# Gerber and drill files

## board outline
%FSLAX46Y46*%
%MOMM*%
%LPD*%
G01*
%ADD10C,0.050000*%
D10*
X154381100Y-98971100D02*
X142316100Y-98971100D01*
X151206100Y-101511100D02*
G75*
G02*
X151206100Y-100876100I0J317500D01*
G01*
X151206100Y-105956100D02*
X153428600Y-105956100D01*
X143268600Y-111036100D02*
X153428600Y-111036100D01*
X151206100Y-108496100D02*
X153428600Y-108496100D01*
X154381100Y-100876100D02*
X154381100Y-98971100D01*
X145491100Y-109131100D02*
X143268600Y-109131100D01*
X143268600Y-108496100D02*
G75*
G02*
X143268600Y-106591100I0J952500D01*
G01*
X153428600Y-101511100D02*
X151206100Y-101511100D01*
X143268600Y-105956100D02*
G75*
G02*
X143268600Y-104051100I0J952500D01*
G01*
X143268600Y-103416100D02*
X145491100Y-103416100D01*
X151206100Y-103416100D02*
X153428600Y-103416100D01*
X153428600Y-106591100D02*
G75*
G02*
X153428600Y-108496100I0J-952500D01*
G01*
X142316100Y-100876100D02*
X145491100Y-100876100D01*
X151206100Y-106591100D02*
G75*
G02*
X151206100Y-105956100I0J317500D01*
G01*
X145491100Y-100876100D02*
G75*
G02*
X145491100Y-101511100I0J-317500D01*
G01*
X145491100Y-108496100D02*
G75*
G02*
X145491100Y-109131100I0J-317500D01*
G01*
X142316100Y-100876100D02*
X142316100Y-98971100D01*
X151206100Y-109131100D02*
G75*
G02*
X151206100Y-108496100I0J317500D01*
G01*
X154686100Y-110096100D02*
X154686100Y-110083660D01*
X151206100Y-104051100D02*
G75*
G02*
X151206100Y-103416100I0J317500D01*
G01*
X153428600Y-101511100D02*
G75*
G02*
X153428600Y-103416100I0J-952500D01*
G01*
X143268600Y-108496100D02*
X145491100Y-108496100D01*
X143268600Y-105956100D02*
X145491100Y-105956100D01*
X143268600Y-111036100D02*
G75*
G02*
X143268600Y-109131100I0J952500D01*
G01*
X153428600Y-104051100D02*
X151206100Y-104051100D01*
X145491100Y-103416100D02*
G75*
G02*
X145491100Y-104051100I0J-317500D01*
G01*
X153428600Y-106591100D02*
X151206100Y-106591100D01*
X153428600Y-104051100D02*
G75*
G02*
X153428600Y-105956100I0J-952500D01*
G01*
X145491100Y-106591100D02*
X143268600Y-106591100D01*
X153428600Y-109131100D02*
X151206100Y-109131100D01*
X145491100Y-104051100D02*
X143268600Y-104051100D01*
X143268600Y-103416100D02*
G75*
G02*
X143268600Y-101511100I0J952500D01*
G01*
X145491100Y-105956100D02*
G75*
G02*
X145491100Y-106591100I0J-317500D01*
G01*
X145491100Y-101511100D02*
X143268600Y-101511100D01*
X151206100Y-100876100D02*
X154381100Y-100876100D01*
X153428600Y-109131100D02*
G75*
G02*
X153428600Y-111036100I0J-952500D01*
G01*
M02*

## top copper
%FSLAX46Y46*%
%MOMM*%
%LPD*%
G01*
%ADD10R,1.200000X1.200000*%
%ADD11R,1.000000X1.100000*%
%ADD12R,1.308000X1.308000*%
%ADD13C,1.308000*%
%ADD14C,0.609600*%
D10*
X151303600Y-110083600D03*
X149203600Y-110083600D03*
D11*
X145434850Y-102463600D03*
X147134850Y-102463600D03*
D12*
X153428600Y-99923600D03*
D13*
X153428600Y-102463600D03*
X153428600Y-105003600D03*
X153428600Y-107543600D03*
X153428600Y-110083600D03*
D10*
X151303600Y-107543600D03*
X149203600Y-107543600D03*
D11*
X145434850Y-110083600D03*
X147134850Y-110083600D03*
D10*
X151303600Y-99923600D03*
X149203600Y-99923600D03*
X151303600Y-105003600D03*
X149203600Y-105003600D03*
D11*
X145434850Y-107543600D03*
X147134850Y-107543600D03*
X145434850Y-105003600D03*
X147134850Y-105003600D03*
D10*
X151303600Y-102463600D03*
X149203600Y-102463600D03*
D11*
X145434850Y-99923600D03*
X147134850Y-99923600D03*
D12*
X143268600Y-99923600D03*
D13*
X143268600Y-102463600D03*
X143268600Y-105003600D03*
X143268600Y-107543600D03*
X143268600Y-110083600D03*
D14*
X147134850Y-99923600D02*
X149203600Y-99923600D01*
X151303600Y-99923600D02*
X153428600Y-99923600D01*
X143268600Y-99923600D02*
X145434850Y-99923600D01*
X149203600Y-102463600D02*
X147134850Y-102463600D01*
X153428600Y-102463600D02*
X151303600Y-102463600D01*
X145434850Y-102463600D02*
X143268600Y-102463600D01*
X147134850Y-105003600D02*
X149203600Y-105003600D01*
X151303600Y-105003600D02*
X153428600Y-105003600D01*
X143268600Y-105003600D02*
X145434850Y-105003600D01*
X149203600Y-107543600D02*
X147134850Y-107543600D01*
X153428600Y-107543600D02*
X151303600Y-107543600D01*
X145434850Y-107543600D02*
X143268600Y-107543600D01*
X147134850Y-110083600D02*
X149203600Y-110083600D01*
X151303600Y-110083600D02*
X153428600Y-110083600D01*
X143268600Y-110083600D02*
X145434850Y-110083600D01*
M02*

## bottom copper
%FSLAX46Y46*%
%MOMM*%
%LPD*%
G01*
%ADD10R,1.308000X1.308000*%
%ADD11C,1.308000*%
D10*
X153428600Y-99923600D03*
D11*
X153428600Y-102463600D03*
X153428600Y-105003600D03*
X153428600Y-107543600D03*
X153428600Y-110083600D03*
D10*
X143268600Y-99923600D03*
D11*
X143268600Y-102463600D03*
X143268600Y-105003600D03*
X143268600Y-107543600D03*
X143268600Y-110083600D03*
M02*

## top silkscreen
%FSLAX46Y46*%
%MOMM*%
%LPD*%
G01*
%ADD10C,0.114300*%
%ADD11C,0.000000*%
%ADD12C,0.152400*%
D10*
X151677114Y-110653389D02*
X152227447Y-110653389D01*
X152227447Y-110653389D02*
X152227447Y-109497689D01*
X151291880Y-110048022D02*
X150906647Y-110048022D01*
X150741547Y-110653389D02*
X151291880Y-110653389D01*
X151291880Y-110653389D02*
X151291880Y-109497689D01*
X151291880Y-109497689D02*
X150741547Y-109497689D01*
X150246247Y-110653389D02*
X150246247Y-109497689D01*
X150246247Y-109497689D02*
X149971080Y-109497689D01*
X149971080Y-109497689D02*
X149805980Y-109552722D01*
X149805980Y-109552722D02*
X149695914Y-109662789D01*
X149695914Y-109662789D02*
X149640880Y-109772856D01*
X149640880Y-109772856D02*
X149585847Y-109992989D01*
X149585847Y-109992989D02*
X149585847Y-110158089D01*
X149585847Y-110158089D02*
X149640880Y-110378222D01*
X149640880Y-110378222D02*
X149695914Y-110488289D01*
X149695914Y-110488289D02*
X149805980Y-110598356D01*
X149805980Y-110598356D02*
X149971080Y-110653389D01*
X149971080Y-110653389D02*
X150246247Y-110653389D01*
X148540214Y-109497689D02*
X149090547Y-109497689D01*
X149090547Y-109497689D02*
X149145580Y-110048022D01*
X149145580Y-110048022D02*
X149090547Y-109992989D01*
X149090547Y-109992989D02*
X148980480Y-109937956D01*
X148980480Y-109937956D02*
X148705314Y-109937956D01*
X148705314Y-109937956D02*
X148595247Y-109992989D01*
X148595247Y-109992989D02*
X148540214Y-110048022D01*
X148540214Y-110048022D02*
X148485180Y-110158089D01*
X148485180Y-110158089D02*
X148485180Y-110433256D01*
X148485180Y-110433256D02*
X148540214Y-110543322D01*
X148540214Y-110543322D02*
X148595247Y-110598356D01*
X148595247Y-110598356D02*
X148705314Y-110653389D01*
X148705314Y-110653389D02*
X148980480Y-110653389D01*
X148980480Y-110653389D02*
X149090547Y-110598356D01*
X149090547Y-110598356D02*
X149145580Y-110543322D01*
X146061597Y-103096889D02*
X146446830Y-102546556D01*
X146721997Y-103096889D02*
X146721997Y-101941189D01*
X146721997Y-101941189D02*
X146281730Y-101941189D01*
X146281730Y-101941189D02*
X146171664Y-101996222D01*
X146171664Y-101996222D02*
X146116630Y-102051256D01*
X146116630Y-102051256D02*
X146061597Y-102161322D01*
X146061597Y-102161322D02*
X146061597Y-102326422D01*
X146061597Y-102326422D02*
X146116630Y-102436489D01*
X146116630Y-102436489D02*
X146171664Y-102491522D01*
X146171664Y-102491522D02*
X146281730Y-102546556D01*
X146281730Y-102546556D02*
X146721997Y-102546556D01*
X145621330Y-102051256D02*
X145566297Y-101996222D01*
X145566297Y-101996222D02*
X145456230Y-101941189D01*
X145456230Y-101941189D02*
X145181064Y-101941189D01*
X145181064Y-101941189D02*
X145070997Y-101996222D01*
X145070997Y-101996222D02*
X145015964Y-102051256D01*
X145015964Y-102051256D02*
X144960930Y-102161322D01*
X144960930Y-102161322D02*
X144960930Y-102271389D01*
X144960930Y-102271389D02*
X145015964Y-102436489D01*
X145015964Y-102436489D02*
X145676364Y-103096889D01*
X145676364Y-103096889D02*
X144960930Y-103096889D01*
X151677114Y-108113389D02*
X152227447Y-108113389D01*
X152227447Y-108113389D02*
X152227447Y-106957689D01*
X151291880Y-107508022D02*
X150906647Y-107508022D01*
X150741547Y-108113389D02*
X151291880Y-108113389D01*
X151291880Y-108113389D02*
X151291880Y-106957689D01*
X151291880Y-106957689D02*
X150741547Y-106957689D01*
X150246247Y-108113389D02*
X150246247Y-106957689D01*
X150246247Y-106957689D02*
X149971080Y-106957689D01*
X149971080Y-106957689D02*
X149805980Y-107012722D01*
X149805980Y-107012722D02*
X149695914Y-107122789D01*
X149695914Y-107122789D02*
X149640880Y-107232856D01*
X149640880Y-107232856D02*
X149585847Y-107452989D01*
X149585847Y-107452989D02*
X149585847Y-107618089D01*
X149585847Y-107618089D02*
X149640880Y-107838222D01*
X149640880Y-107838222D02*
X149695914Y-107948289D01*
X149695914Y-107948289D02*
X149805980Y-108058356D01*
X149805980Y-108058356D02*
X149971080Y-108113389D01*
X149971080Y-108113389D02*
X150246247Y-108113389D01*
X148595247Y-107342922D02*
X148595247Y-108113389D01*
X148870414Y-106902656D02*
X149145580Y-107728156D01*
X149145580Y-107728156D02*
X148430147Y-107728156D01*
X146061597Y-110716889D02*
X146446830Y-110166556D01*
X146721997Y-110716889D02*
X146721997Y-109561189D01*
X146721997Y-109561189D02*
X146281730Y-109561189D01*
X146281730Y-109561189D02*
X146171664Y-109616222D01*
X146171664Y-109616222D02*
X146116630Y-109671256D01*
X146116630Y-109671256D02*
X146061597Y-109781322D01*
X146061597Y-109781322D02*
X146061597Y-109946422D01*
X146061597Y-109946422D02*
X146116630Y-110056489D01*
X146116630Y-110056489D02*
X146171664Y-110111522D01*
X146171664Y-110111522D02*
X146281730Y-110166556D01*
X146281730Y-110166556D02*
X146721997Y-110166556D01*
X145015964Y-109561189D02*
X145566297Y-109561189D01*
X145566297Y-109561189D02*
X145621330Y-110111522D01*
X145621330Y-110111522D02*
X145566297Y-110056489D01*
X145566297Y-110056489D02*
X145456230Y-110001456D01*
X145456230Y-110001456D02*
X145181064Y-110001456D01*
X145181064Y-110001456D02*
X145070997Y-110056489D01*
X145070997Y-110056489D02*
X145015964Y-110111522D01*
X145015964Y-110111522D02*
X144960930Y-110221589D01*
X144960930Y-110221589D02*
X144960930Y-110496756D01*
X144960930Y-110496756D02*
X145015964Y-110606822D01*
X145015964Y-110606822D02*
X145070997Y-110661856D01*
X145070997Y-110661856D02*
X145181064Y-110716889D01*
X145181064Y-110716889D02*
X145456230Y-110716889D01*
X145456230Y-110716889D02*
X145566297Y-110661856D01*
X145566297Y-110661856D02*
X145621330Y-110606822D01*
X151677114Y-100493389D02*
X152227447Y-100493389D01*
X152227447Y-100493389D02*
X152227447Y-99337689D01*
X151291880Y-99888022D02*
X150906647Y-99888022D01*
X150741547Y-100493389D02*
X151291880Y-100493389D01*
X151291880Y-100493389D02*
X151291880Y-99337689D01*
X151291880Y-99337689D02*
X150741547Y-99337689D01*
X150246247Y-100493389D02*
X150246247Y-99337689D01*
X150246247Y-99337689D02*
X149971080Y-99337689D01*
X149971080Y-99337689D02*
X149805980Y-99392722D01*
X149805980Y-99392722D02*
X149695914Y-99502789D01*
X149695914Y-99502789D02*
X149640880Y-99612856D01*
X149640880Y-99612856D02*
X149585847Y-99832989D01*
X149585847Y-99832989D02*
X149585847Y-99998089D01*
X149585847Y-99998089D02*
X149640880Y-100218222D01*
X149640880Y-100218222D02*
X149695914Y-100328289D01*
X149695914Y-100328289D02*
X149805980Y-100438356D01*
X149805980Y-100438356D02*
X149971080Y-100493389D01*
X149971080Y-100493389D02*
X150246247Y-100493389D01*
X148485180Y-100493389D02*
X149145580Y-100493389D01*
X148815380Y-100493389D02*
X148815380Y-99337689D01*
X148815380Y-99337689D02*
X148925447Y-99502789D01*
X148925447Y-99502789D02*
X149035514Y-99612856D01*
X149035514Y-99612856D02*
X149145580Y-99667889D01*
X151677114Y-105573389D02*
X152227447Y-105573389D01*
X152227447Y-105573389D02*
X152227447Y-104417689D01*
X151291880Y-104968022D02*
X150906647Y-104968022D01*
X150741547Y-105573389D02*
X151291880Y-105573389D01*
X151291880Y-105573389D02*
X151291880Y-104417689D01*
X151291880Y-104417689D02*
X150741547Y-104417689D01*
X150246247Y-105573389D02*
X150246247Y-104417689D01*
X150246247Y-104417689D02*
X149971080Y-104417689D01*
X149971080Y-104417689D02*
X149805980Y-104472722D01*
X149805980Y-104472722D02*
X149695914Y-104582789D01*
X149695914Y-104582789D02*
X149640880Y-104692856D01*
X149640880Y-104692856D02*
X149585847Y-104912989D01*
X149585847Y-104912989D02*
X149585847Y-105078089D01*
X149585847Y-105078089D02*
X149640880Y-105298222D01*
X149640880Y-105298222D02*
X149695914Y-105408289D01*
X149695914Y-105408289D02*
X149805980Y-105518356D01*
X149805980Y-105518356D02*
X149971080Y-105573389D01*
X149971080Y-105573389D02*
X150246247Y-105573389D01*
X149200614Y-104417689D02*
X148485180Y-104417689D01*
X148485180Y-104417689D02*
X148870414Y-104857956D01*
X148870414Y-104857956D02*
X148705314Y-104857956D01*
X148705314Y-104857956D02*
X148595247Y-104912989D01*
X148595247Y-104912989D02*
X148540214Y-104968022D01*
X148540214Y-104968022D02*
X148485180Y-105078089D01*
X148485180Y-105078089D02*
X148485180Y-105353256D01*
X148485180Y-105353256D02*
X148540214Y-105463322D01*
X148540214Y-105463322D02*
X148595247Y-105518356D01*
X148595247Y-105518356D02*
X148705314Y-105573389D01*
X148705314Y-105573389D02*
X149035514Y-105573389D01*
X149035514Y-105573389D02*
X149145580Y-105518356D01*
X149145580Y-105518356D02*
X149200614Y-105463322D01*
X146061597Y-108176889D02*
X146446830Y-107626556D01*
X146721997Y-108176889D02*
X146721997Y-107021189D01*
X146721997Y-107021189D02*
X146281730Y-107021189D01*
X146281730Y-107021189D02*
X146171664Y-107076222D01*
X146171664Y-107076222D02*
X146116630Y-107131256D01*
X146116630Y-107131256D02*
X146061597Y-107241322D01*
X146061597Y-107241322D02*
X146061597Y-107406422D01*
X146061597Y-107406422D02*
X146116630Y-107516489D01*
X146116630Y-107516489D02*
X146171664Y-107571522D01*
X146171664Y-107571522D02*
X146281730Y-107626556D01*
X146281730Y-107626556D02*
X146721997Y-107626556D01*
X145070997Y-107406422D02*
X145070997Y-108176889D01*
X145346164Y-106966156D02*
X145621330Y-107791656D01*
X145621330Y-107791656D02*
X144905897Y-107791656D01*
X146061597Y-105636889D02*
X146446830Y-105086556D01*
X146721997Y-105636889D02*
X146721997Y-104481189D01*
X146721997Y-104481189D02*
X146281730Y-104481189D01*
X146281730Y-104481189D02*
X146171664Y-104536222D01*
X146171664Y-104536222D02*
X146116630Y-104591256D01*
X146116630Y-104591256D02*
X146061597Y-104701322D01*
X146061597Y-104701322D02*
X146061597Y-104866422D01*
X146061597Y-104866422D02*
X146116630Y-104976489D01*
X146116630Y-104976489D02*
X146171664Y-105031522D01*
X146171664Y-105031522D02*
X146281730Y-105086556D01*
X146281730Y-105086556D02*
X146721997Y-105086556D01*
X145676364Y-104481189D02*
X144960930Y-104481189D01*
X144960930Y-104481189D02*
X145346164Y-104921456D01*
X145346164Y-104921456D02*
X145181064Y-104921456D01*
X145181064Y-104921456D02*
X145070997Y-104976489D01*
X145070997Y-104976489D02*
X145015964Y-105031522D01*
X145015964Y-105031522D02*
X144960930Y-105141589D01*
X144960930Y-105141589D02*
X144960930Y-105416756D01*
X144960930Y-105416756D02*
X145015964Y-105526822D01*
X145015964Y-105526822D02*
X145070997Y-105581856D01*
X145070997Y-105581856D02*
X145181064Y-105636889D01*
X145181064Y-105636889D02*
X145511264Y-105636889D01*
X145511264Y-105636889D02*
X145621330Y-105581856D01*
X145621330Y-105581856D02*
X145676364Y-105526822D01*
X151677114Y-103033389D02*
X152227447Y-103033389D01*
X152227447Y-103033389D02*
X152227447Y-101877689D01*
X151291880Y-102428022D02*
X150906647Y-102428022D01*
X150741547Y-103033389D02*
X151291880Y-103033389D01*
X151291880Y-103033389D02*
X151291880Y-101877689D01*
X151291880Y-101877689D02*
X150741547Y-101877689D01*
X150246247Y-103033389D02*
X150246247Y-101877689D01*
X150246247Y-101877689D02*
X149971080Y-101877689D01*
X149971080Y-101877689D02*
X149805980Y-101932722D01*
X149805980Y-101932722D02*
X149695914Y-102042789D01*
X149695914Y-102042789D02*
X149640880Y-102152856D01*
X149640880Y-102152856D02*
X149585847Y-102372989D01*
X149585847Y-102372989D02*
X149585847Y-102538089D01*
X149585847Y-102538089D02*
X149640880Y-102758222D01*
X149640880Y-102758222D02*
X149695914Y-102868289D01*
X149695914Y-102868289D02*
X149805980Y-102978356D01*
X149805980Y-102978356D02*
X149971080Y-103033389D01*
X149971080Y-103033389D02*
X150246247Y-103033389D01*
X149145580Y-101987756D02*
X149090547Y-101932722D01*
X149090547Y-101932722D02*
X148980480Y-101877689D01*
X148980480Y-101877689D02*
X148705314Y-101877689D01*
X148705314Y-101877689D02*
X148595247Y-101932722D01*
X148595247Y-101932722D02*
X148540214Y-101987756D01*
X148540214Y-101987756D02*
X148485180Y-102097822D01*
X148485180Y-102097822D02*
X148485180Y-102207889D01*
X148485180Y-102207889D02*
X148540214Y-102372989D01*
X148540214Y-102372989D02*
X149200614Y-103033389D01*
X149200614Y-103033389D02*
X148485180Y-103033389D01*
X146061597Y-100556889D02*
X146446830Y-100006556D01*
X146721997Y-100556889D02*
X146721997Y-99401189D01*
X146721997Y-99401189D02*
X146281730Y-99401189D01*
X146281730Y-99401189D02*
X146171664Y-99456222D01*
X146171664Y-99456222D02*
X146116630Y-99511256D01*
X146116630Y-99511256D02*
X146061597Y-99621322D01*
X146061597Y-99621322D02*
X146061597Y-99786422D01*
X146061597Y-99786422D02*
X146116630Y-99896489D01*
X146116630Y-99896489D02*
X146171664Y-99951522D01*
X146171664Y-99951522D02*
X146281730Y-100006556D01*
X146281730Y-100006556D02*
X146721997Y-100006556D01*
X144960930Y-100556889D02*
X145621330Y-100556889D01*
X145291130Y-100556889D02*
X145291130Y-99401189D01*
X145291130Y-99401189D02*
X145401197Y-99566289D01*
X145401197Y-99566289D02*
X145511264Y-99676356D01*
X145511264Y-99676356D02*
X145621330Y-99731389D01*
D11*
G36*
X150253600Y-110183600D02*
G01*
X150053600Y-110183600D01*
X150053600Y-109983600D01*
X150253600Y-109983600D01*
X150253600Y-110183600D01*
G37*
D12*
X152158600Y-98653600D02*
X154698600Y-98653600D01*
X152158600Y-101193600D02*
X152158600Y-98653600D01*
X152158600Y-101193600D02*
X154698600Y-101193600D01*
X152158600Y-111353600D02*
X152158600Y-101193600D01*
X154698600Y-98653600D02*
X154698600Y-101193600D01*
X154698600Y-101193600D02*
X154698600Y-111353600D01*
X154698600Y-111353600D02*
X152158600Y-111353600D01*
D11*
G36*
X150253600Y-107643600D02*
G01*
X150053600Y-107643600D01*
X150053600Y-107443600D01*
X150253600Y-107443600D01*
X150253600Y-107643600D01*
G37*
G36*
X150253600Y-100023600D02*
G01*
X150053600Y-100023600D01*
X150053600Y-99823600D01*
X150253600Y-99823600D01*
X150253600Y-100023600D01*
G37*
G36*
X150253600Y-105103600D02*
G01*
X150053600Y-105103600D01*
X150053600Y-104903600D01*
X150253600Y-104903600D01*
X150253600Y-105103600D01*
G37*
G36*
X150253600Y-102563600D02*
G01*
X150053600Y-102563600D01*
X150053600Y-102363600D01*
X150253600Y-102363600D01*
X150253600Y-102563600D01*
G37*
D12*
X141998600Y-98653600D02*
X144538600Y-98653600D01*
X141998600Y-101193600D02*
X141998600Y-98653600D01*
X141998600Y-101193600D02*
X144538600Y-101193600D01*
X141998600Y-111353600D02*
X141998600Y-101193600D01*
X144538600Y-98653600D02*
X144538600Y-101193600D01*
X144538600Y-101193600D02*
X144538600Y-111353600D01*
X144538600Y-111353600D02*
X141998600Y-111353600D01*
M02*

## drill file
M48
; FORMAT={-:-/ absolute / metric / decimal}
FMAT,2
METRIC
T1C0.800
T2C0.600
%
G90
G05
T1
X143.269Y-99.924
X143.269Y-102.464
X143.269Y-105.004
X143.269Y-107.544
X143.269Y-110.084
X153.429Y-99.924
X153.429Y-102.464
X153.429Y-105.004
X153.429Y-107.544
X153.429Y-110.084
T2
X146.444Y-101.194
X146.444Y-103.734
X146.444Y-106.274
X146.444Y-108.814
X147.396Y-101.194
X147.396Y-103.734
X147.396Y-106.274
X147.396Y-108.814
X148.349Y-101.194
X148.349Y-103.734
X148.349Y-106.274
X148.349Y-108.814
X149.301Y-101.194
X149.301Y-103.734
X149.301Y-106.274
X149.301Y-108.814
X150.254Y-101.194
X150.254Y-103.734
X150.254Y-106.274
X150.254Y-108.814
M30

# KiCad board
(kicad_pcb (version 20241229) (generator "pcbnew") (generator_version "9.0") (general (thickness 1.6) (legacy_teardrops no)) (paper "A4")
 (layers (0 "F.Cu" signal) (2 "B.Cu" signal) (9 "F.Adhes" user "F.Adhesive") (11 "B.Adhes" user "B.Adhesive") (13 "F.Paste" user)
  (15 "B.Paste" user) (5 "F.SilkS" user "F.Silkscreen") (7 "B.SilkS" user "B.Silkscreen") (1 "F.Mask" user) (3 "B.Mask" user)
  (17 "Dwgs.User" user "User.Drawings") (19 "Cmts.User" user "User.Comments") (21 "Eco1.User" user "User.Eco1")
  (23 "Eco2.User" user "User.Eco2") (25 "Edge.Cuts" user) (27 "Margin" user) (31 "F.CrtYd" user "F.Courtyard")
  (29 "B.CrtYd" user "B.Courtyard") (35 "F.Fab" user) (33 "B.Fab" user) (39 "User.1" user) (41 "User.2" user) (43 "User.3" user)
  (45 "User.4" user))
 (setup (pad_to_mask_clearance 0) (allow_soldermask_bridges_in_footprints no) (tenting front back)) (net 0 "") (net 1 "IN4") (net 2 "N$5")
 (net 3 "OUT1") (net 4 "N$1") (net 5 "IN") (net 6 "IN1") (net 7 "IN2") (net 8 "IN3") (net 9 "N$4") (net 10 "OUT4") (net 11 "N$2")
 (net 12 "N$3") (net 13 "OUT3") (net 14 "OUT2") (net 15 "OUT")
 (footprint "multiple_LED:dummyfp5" (layer "F.Cu") (at 148.3486 103.7336)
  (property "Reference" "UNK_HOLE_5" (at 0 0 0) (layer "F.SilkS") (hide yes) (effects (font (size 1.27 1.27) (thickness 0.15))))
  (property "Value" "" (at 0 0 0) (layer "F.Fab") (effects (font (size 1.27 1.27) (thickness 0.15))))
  (pad "" np_thru_hole circle (at 0 0) (size 0.6 0.6) (drill 0.6) (layers "*.Cu" "*.Mask")))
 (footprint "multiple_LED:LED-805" (layer "F.Cu") (at 150.2536 110.0836 90)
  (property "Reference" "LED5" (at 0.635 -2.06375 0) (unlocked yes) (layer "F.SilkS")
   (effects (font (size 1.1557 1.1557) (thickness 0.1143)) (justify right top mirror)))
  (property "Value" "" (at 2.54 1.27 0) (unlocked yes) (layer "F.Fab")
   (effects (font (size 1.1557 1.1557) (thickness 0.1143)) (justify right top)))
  (fp_poly (pts (xy -0.1 0) (xy 0.1 0) (xy 0.1 -0.2) (xy -0.1 -0.2)) (stroke (width 0) (type default)) (fill yes) (layer "F.SilkS"))
  (pad "A" smd rect (at 0 1.05 90) (size 1.2 1.2) (layers "F.Cu" "F.Mask" "F.Paste") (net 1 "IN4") (solder_mask_margin 0.0508)
   (solder_paste_margin 0) (thermal_bridge_angle 0))
  (pad "C" smd rect (at 0 -1.05 90) (size 1.2 1.2) (layers "F.Cu" "F.Mask" "F.Paste") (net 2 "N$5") (solder_mask_margin 0.0508)
   (solder_paste_margin 0) (thermal_bridge_angle 0)))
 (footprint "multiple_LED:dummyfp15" (layer "F.Cu") (at 148.3486 108.8136)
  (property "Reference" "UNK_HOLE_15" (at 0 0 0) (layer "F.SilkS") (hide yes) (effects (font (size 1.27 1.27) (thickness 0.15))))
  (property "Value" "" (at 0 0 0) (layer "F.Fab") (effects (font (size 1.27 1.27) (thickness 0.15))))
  (pad "" np_thru_hole circle (at 0 0) (size 0.6 0.6) (drill 0.6) (layers "*.Cu" "*.Mask")))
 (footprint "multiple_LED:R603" (layer "F.Cu") (at 146.28485 102.4636)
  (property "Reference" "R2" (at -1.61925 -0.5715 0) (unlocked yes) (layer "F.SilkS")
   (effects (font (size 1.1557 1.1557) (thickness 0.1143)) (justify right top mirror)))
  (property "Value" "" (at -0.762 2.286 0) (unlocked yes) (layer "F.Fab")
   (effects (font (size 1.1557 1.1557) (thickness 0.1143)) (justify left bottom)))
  (pad "1" smd rect (at -0.85 0) (size 1 1.1) (layers "F.Cu" "F.Mask" "F.Paste") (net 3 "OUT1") (solder_mask_margin 0.0508)
   (solder_paste_margin 0) (thermal_bridge_angle 0))
  (pad "2" smd rect (at 0.85 0) (size 1 1.1) (layers "F.Cu" "F.Mask" "F.Paste") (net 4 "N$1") (solder_mask_margin 0.0508)
   (solder_paste_margin 0) (thermal_bridge_angle 0)))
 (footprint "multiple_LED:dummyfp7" (layer "F.Cu") (at 149.3011 103.7336)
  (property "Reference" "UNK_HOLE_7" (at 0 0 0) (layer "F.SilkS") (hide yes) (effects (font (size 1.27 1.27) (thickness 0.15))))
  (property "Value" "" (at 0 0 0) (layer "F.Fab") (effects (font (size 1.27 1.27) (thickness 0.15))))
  (pad "" np_thru_hole circle (at 0 0) (size 0.6 0.6) (drill 0.6) (layers "*.Cu" "*.Mask")))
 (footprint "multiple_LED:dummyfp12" (layer "F.Cu") (at 149.3011 106.2736)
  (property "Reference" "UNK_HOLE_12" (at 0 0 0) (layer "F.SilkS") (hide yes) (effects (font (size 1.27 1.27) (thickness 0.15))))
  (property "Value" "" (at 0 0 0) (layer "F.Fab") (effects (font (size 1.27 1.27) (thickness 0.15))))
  (pad "" np_thru_hole circle (at 0 0) (size 0.6 0.6) (drill 0.6) (layers "*.Cu" "*.Mask")))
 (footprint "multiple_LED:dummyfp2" (layer "F.Cu") (at 149.3011 101.1936)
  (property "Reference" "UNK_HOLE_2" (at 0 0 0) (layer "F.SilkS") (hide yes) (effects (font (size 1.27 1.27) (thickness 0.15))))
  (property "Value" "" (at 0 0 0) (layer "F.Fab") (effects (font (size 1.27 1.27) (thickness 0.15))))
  (pad "" np_thru_hole circle (at 0 0) (size 0.6 0.6) (drill 0.6) (layers "*.Cu" "*.Mask")))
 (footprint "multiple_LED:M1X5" (layer "F.Cu") (at 153.4286 105.0036 -90)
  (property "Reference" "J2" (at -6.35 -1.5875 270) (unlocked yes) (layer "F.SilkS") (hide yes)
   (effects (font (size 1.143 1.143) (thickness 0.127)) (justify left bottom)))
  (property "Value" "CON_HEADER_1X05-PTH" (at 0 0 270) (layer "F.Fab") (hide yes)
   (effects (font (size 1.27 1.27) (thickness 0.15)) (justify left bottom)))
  (fp_line (start -6.35 1.27) (end -6.35 -1.27) (stroke (width 0.1524) (type solid)) (layer "F.SilkS"))
  (fp_line (start -3.81 1.27) (end -6.35 1.27) (stroke (width 0.1524) (type solid)) (layer "F.SilkS"))
  (fp_line (start -3.81 1.27) (end -3.81 -1.27) (stroke (width 0.1524) (type solid)) (layer "F.SilkS"))
  (fp_line (start 6.35 1.27) (end -3.81 1.27) (stroke (width 0.1524) (type solid)) (layer "F.SilkS"))
  (fp_line (start -6.35 -1.27) (end -3.81 -1.27) (stroke (width 0.1524) (type solid)) (layer "F.SilkS"))
  (fp_line (start -3.81 -1.27) (end 6.35 -1.27) (stroke (width 0.1524) (type solid)) (layer "F.SilkS"))
  (fp_line (start 6.35 -1.27) (end 6.35 1.27) (stroke (width 0.1524) (type solid)) (layer "F.SilkS"))
  (pad "1" thru_hole rect (at -5.08 0 270) (size 1.308 1.308) (drill 0.8) (layers "*.Cu" "*.Mask") (remove_unused_layers no) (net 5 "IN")
   (solder_mask_margin 0.0508) (thermal_bridge_angle 0))
  (pad "2" thru_hole circle (at -2.54 0 270) (size 1.308 1.308) (drill 0.8) (layers "*.Cu" "*.Mask") (remove_unused_layers no) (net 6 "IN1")
   (solder_mask_margin 0.0508) (thermal_bridge_angle 0))
  (pad "3" thru_hole circle (at 0 0 270) (size 1.308 1.308) (drill 0.8) (layers "*.Cu" "*.Mask") (remove_unused_layers no) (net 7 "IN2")
   (solder_mask_margin 0.0508) (thermal_bridge_angle 0))
  (pad "4" thru_hole circle (at 2.54 0 270) (size 1.308 1.308) (drill 0.8) (layers "*.Cu" "*.Mask") (remove_unused_layers no) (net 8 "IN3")
   (solder_mask_margin 0.0508) (thermal_bridge_angle 0))
  (pad "5" thru_hole circle (at 5.08 0 270) (size 1.308 1.308) (drill 0.8) (layers "*.Cu" "*.Mask") (remove_unused_layers no) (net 1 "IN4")
   (solder_mask_margin 0.0508) (thermal_bridge_angle 0)))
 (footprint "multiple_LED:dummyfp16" (layer "F.Cu") (at 147.3961 108.8136)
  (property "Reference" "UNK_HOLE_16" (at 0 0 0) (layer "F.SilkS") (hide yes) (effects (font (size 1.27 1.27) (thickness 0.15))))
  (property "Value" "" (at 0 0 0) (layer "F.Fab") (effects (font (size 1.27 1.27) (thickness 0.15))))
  (pad "" np_thru_hole circle (at 0 0) (size 0.6 0.6) (drill 0.6) (layers "*.Cu" "*.Mask")))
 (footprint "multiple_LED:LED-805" (layer "F.Cu") (at 150.2536 107.5436 90)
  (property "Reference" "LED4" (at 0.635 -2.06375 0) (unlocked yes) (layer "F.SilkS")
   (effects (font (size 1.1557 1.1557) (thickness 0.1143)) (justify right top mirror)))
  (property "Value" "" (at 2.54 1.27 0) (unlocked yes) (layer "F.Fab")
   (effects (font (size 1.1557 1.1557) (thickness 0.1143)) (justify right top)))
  (fp_poly (pts (xy -0.1 0) (xy 0.1 0) (xy 0.1 -0.2) (xy -0.1 -0.2)) (stroke (width 0) (type default)) (fill yes) (layer "F.SilkS"))
  (pad "A" smd rect (at 0 1.05 90) (size 1.2 1.2) (layers "F.Cu" "F.Mask" "F.Paste") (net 8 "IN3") (solder_mask_margin 0.0508)
   (solder_paste_margin 0) (thermal_bridge_angle 0))
  (pad "C" smd rect (at 0 -1.05 90) (size 1.2 1.2) (layers "F.Cu" "F.Mask" "F.Paste") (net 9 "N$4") (solder_mask_margin 0.0508)
   (solder_paste_margin 0) (thermal_bridge_angle 0)))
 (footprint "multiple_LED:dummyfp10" (layer "F.Cu") (at 148.3486 106.2736)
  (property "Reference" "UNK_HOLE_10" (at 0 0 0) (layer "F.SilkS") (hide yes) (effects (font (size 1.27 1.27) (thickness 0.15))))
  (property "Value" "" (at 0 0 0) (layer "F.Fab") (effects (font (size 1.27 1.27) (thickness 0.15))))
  (pad "" np_thru_hole circle (at 0 0) (size 0.6 0.6) (drill 0.6) (layers "*.Cu" "*.Mask")))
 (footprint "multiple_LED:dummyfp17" (layer "F.Cu") (at 149.3011 108.8136)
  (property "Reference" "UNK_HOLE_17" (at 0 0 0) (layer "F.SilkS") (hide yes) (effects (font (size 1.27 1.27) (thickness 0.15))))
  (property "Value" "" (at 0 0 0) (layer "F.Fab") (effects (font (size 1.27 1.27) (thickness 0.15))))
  (pad "" np_thru_hole circle (at 0 0) (size 0.6 0.6) (drill 0.6) (layers "*.Cu" "*.Mask")))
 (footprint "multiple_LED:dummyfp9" (layer "F.Cu") (at 146.4436 103.7336)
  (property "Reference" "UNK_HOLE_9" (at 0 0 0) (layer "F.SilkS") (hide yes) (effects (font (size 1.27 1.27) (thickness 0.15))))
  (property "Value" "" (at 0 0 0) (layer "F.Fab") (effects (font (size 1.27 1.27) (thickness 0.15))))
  (pad "" np_thru_hole circle (at 0 0) (size 0.6 0.6) (drill 0.6) (layers "*.Cu" "*.Mask")))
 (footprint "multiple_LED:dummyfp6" (layer "F.Cu") (at 147.3961 103.7336)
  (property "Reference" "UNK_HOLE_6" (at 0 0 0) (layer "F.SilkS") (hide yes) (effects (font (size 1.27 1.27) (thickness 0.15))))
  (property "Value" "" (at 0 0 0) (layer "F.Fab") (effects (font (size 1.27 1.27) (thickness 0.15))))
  (pad "" np_thru_hole circle (at 0 0) (size 0.6 0.6) (drill 0.6) (layers "*.Cu" "*.Mask")))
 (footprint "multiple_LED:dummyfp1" (layer "F.Cu") (at 147.3961 101.1936)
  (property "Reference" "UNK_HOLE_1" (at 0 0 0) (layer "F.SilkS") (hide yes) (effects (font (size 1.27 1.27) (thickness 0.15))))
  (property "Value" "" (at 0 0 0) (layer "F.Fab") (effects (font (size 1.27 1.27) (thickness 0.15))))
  (pad "" np_thru_hole circle (at 0 0) (size 0.6 0.6) (drill 0.6) (layers "*.Cu" "*.Mask")))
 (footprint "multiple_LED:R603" (layer "F.Cu") (at 146.28485 110.0836)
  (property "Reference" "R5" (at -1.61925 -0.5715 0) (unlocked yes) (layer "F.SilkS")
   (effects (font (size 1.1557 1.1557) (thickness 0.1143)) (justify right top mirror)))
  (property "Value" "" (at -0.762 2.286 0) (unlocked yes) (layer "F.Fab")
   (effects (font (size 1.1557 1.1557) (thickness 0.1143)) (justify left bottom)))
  (pad "1" smd rect (at -0.85 0) (size 1 1.1) (layers "F.Cu" "F.Mask" "F.Paste") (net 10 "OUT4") (solder_mask_margin 0.0508)
   (solder_paste_margin 0) (thermal_bridge_angle 0))
  (pad "2" smd rect (at 0.85 0) (size 1 1.1) (layers "F.Cu" "F.Mask" "F.Paste") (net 2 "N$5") (solder_mask_margin 0.0508)
   (solder_paste_margin 0) (thermal_bridge_angle 0)))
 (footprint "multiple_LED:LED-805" (layer "F.Cu") (at 150.2536 99.9236 90)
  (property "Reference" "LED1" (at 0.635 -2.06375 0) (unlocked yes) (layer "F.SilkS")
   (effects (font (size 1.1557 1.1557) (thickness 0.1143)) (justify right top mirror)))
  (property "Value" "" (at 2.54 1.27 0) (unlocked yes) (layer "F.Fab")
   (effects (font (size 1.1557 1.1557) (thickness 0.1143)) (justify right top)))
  (fp_poly (pts (xy -0.1 0) (xy 0.1 0) (xy 0.1 -0.2) (xy -0.1 -0.2)) (stroke (width 0) (type default)) (fill yes) (layer "F.SilkS"))
  (pad "A" smd rect (at 0 1.05 90) (size 1.2 1.2) (layers "F.Cu" "F.Mask" "F.Paste") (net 5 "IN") (solder_mask_margin 0.0508)
   (solder_paste_margin 0) (thermal_bridge_angle 0))
  (pad "C" smd rect (at 0 -1.05 90) (size 1.2 1.2) (layers "F.Cu" "F.Mask" "F.Paste") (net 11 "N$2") (solder_mask_margin 0.0508)
   (solder_paste_margin 0) (thermal_bridge_angle 0)))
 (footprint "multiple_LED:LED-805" (layer "F.Cu") (at 150.2536 105.0036 90)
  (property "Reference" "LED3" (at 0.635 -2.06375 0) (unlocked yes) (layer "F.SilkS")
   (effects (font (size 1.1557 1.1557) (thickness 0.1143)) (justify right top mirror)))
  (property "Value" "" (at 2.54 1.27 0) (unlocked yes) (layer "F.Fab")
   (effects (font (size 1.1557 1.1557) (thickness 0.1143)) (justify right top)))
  (fp_poly (pts (xy -0.1 0) (xy 0.1 0) (xy 0.1 -0.2) (xy -0.1 -0.2)) (stroke (width 0) (type default)) (fill yes) (layer "F.SilkS"))
  (pad "A" smd rect (at 0 1.05 90) (size 1.2 1.2) (layers "F.Cu" "F.Mask" "F.Paste") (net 7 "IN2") (solder_mask_margin 0.0508)
   (solder_paste_margin 0) (thermal_bridge_angle 0))
  (pad "C" smd rect (at 0 -1.05 90) (size 1.2 1.2) (layers "F.Cu" "F.Mask" "F.Paste") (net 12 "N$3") (solder_mask_margin 0.0508)
   (solder_paste_margin 0) (thermal_bridge_angle 0)))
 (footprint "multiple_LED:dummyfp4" (layer "F.Cu") (at 146.4436 101.1936)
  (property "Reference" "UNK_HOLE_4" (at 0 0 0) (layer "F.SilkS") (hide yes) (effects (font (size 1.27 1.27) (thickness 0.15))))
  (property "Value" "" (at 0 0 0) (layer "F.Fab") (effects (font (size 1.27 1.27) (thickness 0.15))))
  (pad "" np_thru_hole circle (at 0 0) (size 0.6 0.6) (drill 0.6) (layers "*.Cu" "*.Mask")))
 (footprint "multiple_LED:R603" (layer "F.Cu") (at 146.28485 107.5436)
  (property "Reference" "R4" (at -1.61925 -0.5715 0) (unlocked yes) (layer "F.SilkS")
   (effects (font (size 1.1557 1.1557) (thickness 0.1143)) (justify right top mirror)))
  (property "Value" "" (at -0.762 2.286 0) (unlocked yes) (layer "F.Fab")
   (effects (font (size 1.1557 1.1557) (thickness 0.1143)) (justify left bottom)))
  (pad "1" smd rect (at -0.85 0) (size 1 1.1) (layers "F.Cu" "F.Mask" "F.Paste") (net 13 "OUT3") (solder_mask_margin 0.0508)
   (solder_paste_margin 0) (thermal_bridge_angle 0))
  (pad "2" smd rect (at 0.85 0) (size 1 1.1) (layers "F.Cu" "F.Mask" "F.Paste") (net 9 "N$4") (solder_mask_margin 0.0508)
   (solder_paste_margin 0) (thermal_bridge_angle 0)))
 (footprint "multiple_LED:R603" (layer "F.Cu") (at 146.28485 105.0036)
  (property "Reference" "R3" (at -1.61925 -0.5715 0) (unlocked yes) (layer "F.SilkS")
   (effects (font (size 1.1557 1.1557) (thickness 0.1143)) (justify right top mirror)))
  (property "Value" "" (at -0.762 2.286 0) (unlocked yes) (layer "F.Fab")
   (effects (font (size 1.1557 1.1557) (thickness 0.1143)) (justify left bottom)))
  (pad "1" smd rect (at -0.85 0) (size 1 1.1) (layers "F.Cu" "F.Mask" "F.Paste") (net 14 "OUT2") (solder_mask_margin 0.0508)
   (solder_paste_margin 0) (thermal_bridge_angle 0))
  (pad "2" smd rect (at 0.85 0) (size 1 1.1) (layers "F.Cu" "F.Mask" "F.Paste") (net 12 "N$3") (solder_mask_margin 0.0508)
   (solder_paste_margin 0) (thermal_bridge_angle 0)))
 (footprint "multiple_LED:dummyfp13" (layer "F.Cu") (at 150.2536 106.2736)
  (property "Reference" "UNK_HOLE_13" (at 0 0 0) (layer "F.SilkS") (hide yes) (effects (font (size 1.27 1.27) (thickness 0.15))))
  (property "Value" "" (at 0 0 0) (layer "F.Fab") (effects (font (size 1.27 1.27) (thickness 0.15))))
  (pad "" np_thru_hole circle (at 0 0) (size 0.6 0.6) (drill 0.6) (layers "*.Cu" "*.Mask")))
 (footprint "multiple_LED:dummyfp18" (layer "F.Cu") (at 150.2536 108.8136)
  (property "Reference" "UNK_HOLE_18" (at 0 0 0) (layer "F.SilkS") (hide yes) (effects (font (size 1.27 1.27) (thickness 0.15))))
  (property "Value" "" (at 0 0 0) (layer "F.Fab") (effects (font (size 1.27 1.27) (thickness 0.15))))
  (pad "" np_thru_hole circle (at 0 0) (size 0.6 0.6) (drill 0.6) (layers "*.Cu" "*.Mask")))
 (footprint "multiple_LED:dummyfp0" (layer "F.Cu") (at 148.3486 101.1936)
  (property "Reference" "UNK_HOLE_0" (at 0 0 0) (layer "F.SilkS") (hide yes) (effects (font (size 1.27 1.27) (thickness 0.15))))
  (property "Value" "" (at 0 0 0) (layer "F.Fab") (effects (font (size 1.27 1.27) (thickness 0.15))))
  (pad "" np_thru_hole circle (at 0 0) (size 0.6 0.6) (drill 0.6) (layers "*.Cu" "*.Mask")))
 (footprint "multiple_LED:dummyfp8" (layer "F.Cu") (at 150.2536 103.7336)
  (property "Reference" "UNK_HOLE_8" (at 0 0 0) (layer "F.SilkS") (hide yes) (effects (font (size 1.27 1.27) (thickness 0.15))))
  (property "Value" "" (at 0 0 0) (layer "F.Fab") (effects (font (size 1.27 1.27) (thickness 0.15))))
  (pad "" np_thru_hole circle (at 0 0) (size 0.6 0.6) (drill 0.6) (layers "*.Cu" "*.Mask")))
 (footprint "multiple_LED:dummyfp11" (layer "F.Cu") (at 147.3961 106.2736)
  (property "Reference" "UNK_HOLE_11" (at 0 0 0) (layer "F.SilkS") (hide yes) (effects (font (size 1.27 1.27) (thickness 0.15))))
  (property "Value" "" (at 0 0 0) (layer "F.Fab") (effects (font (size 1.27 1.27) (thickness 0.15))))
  (pad "" np_thru_hole circle (at 0 0) (size 0.6 0.6) (drill 0.6) (layers "*.Cu" "*.Mask")))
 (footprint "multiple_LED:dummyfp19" (layer "F.Cu") (at 146.4436 108.8136)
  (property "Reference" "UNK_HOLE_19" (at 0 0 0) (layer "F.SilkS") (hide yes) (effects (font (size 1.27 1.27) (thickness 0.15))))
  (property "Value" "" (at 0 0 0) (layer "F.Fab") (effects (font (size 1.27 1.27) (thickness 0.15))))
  (pad "" np_thru_hole circle (at 0 0) (size 0.6 0.6) (drill 0.6) (layers "*.Cu" "*.Mask")))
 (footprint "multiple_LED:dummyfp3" (layer "F.Cu") (at 150.2536 101.1936)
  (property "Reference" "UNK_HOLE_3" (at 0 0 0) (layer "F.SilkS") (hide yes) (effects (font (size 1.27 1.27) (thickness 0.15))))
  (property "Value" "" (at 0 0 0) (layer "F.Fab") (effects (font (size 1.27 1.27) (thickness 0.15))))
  (pad "" np_thru_hole circle (at 0 0) (size 0.6 0.6) (drill 0.6) (layers "*.Cu" "*.Mask")))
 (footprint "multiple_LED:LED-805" (layer "F.Cu") (at 150.2536 102.4636 90)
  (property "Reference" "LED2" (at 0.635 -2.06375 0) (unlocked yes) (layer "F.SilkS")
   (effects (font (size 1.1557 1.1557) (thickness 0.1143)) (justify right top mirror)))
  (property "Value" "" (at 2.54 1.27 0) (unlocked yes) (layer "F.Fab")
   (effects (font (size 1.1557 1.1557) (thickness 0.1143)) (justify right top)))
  (fp_poly (pts (xy -0.1 0) (xy 0.1 0) (xy 0.1 -0.2) (xy -0.1 -0.2)) (stroke (width 0) (type default)) (fill yes) (layer "F.SilkS"))
  (pad "A" smd rect (at 0 1.05 90) (size 1.2 1.2) (layers "F.Cu" "F.Mask" "F.Paste") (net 6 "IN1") (solder_mask_margin 0.0508)
   (solder_paste_margin 0) (thermal_bridge_angle 0))
  (pad "C" smd rect (at 0 -1.05 90) (size 1.2 1.2) (layers "F.Cu" "F.Mask" "F.Paste") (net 4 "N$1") (solder_mask_margin 0.0508)
   (solder_paste_margin 0) (thermal_bridge_angle 0)))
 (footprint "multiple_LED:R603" (layer "F.Cu") (at 146.28485 99.9236)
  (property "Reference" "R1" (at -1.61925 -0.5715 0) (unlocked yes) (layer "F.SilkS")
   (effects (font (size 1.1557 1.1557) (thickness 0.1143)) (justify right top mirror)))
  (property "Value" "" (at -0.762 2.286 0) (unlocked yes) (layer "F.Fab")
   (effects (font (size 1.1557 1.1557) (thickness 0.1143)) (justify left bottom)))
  (pad "1" smd rect (at -0.85 0) (size 1 1.1) (layers "F.Cu" "F.Mask" "F.Paste") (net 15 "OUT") (solder_mask_margin 0.0508)
   (solder_paste_margin 0) (thermal_bridge_angle 0))
  (pad "2" smd rect (at 0.85 0) (size 1 1.1) (layers "F.Cu" "F.Mask" "F.Paste") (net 11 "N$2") (solder_mask_margin 0.0508)
   (solder_paste_margin 0) (thermal_bridge_angle 0)))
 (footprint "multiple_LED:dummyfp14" (layer "F.Cu") (at 146.4436 106.2736)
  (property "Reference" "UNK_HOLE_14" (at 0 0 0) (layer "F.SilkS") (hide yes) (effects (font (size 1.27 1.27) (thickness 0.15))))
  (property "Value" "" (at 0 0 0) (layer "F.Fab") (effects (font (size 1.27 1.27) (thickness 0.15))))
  (pad "" np_thru_hole circle (at 0 0) (size 0.6 0.6) (drill 0.6) (layers "*.Cu" "*.Mask")))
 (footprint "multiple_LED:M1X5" (layer "F.Cu") (at 143.2686 105.0036 -90)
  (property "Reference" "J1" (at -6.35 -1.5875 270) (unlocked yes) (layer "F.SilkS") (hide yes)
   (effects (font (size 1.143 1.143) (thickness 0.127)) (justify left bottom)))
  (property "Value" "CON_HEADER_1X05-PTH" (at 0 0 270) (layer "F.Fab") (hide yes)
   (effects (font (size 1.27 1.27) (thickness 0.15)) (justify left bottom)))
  (fp_line (start -6.35 1.27) (end -6.35 -1.27) (stroke (width 0.1524) (type solid)) (layer "F.SilkS"))
  (fp_line (start -3.81 1.27) (end -6.35 1.27) (stroke (width 0.1524) (type solid)) (layer "F.SilkS"))
  (fp_line (start -3.81 1.27) (end -3.81 -1.27) (stroke (width 0.1524) (type solid)) (layer "F.SilkS"))
  (fp_line (start 6.35 1.27) (end -3.81 1.27) (stroke (width 0.1524) (type solid)) (layer "F.SilkS"))
  (fp_line (start -6.35 -1.27) (end -3.81 -1.27) (stroke (width 0.1524) (type solid)) (layer "F.SilkS"))
  (fp_line (start -3.81 -1.27) (end 6.35 -1.27) (stroke (width 0.1524) (type solid)) (layer "F.SilkS"))
  (fp_line (start 6.35 -1.27) (end 6.35 1.27) (stroke (width 0.1524) (type solid)) (layer "F.SilkS"))
  (pad "1" thru_hole rect (at -5.08 0 270) (size 1.308 1.308) (drill 0.8) (layers "*.Cu" "*.Mask") (remove_unused_layers no) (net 15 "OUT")
   (solder_mask_margin 0.0508) (thermal_bridge_angle 0))
  (pad "2" thru_hole circle (at -2.54 0 270) (size 1.308 1.308) (drill 0.8) (layers "*.Cu" "*.Mask") (remove_unused_layers no)
   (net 3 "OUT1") (solder_mask_margin 0.0508) (thermal_bridge_angle 0))
  (pad "3" thru_hole circle (at 0 0 270) (size 1.308 1.308) (drill 0.8) (layers "*.Cu" "*.Mask") (remove_unused_layers no) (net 14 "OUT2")
   (solder_mask_margin 0.0508) (thermal_bridge_angle 0))
  (pad "4" thru_hole circle (at 2.54 0 270) (size 1.308 1.308) (drill 0.8) (layers "*.Cu" "*.Mask") (remove_unused_layers no)
   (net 13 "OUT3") (solder_mask_margin 0.0508) (thermal_bridge_angle 0))
  (pad "5" thru_hole circle (at 5.08 0 270) (size 1.308 1.308) (drill 0.8) (layers "*.Cu" "*.Mask") (remove_unused_layers no)
   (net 10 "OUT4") (solder_mask_margin 0.0508) (thermal_bridge_angle 0)))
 (gr_line (start 154.3811 98.9711) (end 142.3161 98.9711) (stroke (width 0.05) (type solid)) (layer "Edge.Cuts"))
 (gr_arc (start 151.2061 101.5111) (mid 150.8886 101.1936) (end 151.2061 100.8761) (stroke (width 0.05) (type solid)) (layer "Edge.Cuts"))
 (gr_line (start 151.2061 105.9561) (end 153.4286 105.9561) (stroke (width 0.05) (type solid)) (layer "Edge.Cuts"))
 (gr_line (start 143.2686 111.0361) (end 153.4286 111.0361) (stroke (width 0.05) (type solid)) (layer "Edge.Cuts"))
 (gr_line (start 151.2061 108.4961) (end 153.4286 108.4961) (stroke (width 0.05) (type solid)) (layer "Edge.Cuts"))
 (gr_line (start 154.3811 100.8761) (end 154.3811 98.9711) (stroke (width 0.05) (type solid)) (layer "Edge.Cuts"))
 (gr_line (start 145.4911 109.1311) (end 143.2686 109.1311) (stroke (width 0.05) (type solid)) (layer "Edge.Cuts"))
 (gr_arc (start 143.2686 108.4961) (mid 142.3161 107.5436) (end 143.2686 106.5911) (stroke (width 0.05) (type solid)) (layer "Edge.Cuts"))
 (gr_line (start 153.4286 101.5111) (end 151.2061 101.5111) (stroke (width 0.05) (type solid)) (layer "Edge.Cuts"))
 (gr_arc (start 143.2686 105.9561) (mid 142.3161 105.0036) (end 143.2686 104.0511) (stroke (width 0.05) (type solid)) (layer "Edge.Cuts"))
 (gr_line (start 143.2686 103.4161) (end 145.4911 103.4161) (stroke (width 0.05) (type solid)) (layer "Edge.Cuts"))
 (gr_line (start 151.2061 103.4161) (end 153.4286 103.4161) (stroke (width 0.05) (type solid)) (layer "Edge.Cuts"))
 (gr_arc (start 153.4286 106.5911) (mid 154.3811 107.5436) (end 153.4286 108.4961) (stroke (width 0.05) (type solid)) (layer "Edge.Cuts"))
 (gr_line (start 142.3161 100.8761) (end 145.4911 100.8761) (stroke (width 0.05) (type solid)) (layer "Edge.Cuts"))
 (gr_arc (start 151.2061 106.5911) (mid 150.8886 106.2736) (end 151.2061 105.9561) (stroke (width 0.05) (type solid)) (layer "Edge.Cuts"))
 (gr_arc (start 145.4911 100.8761) (mid 145.8086 101.1936) (end 145.4911 101.5111) (stroke (width 0.05) (type solid)) (layer "Edge.Cuts"))
 (gr_arc (start 145.4911 108.4961) (mid 145.8086 108.8136) (end 145.4911 109.1311) (stroke (width 0.05) (type solid)) (layer "Edge.Cuts"))
 (gr_line (start 142.3161 100.8761) (end 142.3161 98.9711) (stroke (width 0.05) (type solid)) (layer "Edge.Cuts"))
 (gr_arc (start 151.2061 109.1311) (mid 150.8886 108.8136) (end 151.2061 108.4961) (stroke (width 0.05) (type solid)) (layer "Edge.Cuts"))
 (gr_line (start 154.6861 110.0961) (end 154.6861 110.08366) (stroke (width 0.05) (type solid)) (layer "Edge.Cuts"))
 (gr_arc (start 151.2061 104.0511) (mid 150.8886 103.7336) (end 151.2061 103.4161) (stroke (width 0.05) (type solid)) (layer "Edge.Cuts"))
 (gr_arc (start 153.4286 101.5111) (mid 154.3811 102.4636) (end 153.4286 103.4161) (stroke (width 0.05) (type solid)) (layer "Edge.Cuts"))
 (gr_line (start 143.2686 108.4961) (end 145.4911 108.4961) (stroke (width 0.05) (type solid)) (layer "Edge.Cuts"))
 (gr_line (start 143.2686 105.9561) (end 145.4911 105.9561) (stroke (width 0.05) (type solid)) (layer "Edge.Cuts"))
 (gr_arc (start 143.2686 111.0361) (mid 142.3161 110.0836) (end 143.2686 109.1311) (stroke (width 0.05) (type solid)) (layer "Edge.Cuts"))
 (gr_line (start 153.4286 104.0511) (end 151.2061 104.0511) (stroke (width 0.05) (type solid)) (layer "Edge.Cuts"))
 (gr_arc (start 145.4911 103.4161) (mid 145.8086 103.7336) (end 145.4911 104.0511) (stroke (width 0.05) (type solid)) (layer "Edge.Cuts"))
 (gr_line (start 153.4286 106.5911) (end 151.2061 106.5911) (stroke (width 0.05) (type solid)) (layer "Edge.Cuts"))
 (gr_arc (start 153.4286 104.0511) (mid 154.3811 105.0036) (end 153.4286 105.9561) (stroke (width 0.05) (type solid)) (layer "Edge.Cuts"))
 (gr_line (start 145.4911 106.5911) (end 143.2686 106.5911) (stroke (width 0.05) (type solid)) (layer "Edge.Cuts"))
 (gr_line (start 153.4286 109.1311) (end 151.2061 109.1311) (stroke (width 0.05) (type solid)) (layer "Edge.Cuts"))
 (gr_line (start 145.4911 104.0511) (end 143.2686 104.0511) (stroke (width 0.05) (type solid)) (layer "Edge.Cuts"))
 (gr_arc (start 143.2686 103.4161) (mid 142.3161 102.4636) (end 143.2686 101.5111) (stroke (width 0.05) (type solid)) (layer "Edge.Cuts"))
 (gr_arc (start 145.4911 105.9561) (mid 145.8086 106.2736) (end 145.4911 106.5911) (stroke (width 0.05) (type solid)) (layer "Edge.Cuts"))
 (gr_line (start 145.4911 101.5111) (end 143.2686 101.5111) (stroke (width 0.05) (type solid)) (layer "Edge.Cuts"))
 (gr_line (start 151.2061 100.8761) (end 154.3811 100.8761) (stroke (width 0.05) (type solid)) (layer "Edge.Cuts"))
 (gr_arc (start 153.4286 109.1311) (mid 154.3811 110.0836) (end 153.4286 111.0361) (stroke (width 0.05) (type solid)) (layer "Edge.Cuts"))
 (segment (start 147.13485 99.9236) (end 149.2036 99.9236) (width 0.6096) (layer "F.Cu") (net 11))
 (segment (start 151.3036 99.9236) (end 153.4286 99.9236) (width 0.6096) (layer "F.Cu") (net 5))
 (segment (start 143.2686 99.9236) (end 145.43485 99.9236) (width 0.6096) (layer "F.Cu") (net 15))
 (segment (start 149.2036 102.4636) (end 147.13485 102.4636) (width 0.6096) (layer "F.Cu") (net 4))
 (segment (start 153.4286 102.4636) (end 151.3036 102.4636) (width 0.6096) (layer "F.Cu") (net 6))
 (segment (start 145.43485 102.4636) (end 143.2686 102.4636) (width 0.6096) (layer "F.Cu") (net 3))
 (segment (start 147.13485 105.0036) (end 149.2036 105.0036) (width 0.6096) (layer "F.Cu") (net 12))
 (segment (start 151.3036 105.0036) (end 153.4286 105.0036) (width 0.6096) (layer "F.Cu") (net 7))
 (segment (start 143.2686 105.0036) (end 145.43485 105.0036) (width 0.6096) (layer "F.Cu") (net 14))
 (segment (start 149.2036 107.5436) (end 147.13485 107.5436) (width 0.6096) (layer "F.Cu") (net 9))
 (segment (start 153.4286 107.5436) (end 151.3036 107.5436) (width 0.6096) (layer "F.Cu") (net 8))
 (segment (start 145.43485 107.5436) (end 143.2686 107.5436) (width 0.6096) (layer "F.Cu") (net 13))
 (segment (start 147.13485 110.0836) (end 149.2036 110.0836) (width 0.6096) (layer "F.Cu") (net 2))
 (segment (start 151.3036 110.0836) (end 153.4286 110.0836) (width 0.6096) (layer "F.Cu") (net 1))
 (segment (start 143.2686 110.0836) (end 145.43485 110.0836) (width 0.6096) (layer "F.Cu") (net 10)))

